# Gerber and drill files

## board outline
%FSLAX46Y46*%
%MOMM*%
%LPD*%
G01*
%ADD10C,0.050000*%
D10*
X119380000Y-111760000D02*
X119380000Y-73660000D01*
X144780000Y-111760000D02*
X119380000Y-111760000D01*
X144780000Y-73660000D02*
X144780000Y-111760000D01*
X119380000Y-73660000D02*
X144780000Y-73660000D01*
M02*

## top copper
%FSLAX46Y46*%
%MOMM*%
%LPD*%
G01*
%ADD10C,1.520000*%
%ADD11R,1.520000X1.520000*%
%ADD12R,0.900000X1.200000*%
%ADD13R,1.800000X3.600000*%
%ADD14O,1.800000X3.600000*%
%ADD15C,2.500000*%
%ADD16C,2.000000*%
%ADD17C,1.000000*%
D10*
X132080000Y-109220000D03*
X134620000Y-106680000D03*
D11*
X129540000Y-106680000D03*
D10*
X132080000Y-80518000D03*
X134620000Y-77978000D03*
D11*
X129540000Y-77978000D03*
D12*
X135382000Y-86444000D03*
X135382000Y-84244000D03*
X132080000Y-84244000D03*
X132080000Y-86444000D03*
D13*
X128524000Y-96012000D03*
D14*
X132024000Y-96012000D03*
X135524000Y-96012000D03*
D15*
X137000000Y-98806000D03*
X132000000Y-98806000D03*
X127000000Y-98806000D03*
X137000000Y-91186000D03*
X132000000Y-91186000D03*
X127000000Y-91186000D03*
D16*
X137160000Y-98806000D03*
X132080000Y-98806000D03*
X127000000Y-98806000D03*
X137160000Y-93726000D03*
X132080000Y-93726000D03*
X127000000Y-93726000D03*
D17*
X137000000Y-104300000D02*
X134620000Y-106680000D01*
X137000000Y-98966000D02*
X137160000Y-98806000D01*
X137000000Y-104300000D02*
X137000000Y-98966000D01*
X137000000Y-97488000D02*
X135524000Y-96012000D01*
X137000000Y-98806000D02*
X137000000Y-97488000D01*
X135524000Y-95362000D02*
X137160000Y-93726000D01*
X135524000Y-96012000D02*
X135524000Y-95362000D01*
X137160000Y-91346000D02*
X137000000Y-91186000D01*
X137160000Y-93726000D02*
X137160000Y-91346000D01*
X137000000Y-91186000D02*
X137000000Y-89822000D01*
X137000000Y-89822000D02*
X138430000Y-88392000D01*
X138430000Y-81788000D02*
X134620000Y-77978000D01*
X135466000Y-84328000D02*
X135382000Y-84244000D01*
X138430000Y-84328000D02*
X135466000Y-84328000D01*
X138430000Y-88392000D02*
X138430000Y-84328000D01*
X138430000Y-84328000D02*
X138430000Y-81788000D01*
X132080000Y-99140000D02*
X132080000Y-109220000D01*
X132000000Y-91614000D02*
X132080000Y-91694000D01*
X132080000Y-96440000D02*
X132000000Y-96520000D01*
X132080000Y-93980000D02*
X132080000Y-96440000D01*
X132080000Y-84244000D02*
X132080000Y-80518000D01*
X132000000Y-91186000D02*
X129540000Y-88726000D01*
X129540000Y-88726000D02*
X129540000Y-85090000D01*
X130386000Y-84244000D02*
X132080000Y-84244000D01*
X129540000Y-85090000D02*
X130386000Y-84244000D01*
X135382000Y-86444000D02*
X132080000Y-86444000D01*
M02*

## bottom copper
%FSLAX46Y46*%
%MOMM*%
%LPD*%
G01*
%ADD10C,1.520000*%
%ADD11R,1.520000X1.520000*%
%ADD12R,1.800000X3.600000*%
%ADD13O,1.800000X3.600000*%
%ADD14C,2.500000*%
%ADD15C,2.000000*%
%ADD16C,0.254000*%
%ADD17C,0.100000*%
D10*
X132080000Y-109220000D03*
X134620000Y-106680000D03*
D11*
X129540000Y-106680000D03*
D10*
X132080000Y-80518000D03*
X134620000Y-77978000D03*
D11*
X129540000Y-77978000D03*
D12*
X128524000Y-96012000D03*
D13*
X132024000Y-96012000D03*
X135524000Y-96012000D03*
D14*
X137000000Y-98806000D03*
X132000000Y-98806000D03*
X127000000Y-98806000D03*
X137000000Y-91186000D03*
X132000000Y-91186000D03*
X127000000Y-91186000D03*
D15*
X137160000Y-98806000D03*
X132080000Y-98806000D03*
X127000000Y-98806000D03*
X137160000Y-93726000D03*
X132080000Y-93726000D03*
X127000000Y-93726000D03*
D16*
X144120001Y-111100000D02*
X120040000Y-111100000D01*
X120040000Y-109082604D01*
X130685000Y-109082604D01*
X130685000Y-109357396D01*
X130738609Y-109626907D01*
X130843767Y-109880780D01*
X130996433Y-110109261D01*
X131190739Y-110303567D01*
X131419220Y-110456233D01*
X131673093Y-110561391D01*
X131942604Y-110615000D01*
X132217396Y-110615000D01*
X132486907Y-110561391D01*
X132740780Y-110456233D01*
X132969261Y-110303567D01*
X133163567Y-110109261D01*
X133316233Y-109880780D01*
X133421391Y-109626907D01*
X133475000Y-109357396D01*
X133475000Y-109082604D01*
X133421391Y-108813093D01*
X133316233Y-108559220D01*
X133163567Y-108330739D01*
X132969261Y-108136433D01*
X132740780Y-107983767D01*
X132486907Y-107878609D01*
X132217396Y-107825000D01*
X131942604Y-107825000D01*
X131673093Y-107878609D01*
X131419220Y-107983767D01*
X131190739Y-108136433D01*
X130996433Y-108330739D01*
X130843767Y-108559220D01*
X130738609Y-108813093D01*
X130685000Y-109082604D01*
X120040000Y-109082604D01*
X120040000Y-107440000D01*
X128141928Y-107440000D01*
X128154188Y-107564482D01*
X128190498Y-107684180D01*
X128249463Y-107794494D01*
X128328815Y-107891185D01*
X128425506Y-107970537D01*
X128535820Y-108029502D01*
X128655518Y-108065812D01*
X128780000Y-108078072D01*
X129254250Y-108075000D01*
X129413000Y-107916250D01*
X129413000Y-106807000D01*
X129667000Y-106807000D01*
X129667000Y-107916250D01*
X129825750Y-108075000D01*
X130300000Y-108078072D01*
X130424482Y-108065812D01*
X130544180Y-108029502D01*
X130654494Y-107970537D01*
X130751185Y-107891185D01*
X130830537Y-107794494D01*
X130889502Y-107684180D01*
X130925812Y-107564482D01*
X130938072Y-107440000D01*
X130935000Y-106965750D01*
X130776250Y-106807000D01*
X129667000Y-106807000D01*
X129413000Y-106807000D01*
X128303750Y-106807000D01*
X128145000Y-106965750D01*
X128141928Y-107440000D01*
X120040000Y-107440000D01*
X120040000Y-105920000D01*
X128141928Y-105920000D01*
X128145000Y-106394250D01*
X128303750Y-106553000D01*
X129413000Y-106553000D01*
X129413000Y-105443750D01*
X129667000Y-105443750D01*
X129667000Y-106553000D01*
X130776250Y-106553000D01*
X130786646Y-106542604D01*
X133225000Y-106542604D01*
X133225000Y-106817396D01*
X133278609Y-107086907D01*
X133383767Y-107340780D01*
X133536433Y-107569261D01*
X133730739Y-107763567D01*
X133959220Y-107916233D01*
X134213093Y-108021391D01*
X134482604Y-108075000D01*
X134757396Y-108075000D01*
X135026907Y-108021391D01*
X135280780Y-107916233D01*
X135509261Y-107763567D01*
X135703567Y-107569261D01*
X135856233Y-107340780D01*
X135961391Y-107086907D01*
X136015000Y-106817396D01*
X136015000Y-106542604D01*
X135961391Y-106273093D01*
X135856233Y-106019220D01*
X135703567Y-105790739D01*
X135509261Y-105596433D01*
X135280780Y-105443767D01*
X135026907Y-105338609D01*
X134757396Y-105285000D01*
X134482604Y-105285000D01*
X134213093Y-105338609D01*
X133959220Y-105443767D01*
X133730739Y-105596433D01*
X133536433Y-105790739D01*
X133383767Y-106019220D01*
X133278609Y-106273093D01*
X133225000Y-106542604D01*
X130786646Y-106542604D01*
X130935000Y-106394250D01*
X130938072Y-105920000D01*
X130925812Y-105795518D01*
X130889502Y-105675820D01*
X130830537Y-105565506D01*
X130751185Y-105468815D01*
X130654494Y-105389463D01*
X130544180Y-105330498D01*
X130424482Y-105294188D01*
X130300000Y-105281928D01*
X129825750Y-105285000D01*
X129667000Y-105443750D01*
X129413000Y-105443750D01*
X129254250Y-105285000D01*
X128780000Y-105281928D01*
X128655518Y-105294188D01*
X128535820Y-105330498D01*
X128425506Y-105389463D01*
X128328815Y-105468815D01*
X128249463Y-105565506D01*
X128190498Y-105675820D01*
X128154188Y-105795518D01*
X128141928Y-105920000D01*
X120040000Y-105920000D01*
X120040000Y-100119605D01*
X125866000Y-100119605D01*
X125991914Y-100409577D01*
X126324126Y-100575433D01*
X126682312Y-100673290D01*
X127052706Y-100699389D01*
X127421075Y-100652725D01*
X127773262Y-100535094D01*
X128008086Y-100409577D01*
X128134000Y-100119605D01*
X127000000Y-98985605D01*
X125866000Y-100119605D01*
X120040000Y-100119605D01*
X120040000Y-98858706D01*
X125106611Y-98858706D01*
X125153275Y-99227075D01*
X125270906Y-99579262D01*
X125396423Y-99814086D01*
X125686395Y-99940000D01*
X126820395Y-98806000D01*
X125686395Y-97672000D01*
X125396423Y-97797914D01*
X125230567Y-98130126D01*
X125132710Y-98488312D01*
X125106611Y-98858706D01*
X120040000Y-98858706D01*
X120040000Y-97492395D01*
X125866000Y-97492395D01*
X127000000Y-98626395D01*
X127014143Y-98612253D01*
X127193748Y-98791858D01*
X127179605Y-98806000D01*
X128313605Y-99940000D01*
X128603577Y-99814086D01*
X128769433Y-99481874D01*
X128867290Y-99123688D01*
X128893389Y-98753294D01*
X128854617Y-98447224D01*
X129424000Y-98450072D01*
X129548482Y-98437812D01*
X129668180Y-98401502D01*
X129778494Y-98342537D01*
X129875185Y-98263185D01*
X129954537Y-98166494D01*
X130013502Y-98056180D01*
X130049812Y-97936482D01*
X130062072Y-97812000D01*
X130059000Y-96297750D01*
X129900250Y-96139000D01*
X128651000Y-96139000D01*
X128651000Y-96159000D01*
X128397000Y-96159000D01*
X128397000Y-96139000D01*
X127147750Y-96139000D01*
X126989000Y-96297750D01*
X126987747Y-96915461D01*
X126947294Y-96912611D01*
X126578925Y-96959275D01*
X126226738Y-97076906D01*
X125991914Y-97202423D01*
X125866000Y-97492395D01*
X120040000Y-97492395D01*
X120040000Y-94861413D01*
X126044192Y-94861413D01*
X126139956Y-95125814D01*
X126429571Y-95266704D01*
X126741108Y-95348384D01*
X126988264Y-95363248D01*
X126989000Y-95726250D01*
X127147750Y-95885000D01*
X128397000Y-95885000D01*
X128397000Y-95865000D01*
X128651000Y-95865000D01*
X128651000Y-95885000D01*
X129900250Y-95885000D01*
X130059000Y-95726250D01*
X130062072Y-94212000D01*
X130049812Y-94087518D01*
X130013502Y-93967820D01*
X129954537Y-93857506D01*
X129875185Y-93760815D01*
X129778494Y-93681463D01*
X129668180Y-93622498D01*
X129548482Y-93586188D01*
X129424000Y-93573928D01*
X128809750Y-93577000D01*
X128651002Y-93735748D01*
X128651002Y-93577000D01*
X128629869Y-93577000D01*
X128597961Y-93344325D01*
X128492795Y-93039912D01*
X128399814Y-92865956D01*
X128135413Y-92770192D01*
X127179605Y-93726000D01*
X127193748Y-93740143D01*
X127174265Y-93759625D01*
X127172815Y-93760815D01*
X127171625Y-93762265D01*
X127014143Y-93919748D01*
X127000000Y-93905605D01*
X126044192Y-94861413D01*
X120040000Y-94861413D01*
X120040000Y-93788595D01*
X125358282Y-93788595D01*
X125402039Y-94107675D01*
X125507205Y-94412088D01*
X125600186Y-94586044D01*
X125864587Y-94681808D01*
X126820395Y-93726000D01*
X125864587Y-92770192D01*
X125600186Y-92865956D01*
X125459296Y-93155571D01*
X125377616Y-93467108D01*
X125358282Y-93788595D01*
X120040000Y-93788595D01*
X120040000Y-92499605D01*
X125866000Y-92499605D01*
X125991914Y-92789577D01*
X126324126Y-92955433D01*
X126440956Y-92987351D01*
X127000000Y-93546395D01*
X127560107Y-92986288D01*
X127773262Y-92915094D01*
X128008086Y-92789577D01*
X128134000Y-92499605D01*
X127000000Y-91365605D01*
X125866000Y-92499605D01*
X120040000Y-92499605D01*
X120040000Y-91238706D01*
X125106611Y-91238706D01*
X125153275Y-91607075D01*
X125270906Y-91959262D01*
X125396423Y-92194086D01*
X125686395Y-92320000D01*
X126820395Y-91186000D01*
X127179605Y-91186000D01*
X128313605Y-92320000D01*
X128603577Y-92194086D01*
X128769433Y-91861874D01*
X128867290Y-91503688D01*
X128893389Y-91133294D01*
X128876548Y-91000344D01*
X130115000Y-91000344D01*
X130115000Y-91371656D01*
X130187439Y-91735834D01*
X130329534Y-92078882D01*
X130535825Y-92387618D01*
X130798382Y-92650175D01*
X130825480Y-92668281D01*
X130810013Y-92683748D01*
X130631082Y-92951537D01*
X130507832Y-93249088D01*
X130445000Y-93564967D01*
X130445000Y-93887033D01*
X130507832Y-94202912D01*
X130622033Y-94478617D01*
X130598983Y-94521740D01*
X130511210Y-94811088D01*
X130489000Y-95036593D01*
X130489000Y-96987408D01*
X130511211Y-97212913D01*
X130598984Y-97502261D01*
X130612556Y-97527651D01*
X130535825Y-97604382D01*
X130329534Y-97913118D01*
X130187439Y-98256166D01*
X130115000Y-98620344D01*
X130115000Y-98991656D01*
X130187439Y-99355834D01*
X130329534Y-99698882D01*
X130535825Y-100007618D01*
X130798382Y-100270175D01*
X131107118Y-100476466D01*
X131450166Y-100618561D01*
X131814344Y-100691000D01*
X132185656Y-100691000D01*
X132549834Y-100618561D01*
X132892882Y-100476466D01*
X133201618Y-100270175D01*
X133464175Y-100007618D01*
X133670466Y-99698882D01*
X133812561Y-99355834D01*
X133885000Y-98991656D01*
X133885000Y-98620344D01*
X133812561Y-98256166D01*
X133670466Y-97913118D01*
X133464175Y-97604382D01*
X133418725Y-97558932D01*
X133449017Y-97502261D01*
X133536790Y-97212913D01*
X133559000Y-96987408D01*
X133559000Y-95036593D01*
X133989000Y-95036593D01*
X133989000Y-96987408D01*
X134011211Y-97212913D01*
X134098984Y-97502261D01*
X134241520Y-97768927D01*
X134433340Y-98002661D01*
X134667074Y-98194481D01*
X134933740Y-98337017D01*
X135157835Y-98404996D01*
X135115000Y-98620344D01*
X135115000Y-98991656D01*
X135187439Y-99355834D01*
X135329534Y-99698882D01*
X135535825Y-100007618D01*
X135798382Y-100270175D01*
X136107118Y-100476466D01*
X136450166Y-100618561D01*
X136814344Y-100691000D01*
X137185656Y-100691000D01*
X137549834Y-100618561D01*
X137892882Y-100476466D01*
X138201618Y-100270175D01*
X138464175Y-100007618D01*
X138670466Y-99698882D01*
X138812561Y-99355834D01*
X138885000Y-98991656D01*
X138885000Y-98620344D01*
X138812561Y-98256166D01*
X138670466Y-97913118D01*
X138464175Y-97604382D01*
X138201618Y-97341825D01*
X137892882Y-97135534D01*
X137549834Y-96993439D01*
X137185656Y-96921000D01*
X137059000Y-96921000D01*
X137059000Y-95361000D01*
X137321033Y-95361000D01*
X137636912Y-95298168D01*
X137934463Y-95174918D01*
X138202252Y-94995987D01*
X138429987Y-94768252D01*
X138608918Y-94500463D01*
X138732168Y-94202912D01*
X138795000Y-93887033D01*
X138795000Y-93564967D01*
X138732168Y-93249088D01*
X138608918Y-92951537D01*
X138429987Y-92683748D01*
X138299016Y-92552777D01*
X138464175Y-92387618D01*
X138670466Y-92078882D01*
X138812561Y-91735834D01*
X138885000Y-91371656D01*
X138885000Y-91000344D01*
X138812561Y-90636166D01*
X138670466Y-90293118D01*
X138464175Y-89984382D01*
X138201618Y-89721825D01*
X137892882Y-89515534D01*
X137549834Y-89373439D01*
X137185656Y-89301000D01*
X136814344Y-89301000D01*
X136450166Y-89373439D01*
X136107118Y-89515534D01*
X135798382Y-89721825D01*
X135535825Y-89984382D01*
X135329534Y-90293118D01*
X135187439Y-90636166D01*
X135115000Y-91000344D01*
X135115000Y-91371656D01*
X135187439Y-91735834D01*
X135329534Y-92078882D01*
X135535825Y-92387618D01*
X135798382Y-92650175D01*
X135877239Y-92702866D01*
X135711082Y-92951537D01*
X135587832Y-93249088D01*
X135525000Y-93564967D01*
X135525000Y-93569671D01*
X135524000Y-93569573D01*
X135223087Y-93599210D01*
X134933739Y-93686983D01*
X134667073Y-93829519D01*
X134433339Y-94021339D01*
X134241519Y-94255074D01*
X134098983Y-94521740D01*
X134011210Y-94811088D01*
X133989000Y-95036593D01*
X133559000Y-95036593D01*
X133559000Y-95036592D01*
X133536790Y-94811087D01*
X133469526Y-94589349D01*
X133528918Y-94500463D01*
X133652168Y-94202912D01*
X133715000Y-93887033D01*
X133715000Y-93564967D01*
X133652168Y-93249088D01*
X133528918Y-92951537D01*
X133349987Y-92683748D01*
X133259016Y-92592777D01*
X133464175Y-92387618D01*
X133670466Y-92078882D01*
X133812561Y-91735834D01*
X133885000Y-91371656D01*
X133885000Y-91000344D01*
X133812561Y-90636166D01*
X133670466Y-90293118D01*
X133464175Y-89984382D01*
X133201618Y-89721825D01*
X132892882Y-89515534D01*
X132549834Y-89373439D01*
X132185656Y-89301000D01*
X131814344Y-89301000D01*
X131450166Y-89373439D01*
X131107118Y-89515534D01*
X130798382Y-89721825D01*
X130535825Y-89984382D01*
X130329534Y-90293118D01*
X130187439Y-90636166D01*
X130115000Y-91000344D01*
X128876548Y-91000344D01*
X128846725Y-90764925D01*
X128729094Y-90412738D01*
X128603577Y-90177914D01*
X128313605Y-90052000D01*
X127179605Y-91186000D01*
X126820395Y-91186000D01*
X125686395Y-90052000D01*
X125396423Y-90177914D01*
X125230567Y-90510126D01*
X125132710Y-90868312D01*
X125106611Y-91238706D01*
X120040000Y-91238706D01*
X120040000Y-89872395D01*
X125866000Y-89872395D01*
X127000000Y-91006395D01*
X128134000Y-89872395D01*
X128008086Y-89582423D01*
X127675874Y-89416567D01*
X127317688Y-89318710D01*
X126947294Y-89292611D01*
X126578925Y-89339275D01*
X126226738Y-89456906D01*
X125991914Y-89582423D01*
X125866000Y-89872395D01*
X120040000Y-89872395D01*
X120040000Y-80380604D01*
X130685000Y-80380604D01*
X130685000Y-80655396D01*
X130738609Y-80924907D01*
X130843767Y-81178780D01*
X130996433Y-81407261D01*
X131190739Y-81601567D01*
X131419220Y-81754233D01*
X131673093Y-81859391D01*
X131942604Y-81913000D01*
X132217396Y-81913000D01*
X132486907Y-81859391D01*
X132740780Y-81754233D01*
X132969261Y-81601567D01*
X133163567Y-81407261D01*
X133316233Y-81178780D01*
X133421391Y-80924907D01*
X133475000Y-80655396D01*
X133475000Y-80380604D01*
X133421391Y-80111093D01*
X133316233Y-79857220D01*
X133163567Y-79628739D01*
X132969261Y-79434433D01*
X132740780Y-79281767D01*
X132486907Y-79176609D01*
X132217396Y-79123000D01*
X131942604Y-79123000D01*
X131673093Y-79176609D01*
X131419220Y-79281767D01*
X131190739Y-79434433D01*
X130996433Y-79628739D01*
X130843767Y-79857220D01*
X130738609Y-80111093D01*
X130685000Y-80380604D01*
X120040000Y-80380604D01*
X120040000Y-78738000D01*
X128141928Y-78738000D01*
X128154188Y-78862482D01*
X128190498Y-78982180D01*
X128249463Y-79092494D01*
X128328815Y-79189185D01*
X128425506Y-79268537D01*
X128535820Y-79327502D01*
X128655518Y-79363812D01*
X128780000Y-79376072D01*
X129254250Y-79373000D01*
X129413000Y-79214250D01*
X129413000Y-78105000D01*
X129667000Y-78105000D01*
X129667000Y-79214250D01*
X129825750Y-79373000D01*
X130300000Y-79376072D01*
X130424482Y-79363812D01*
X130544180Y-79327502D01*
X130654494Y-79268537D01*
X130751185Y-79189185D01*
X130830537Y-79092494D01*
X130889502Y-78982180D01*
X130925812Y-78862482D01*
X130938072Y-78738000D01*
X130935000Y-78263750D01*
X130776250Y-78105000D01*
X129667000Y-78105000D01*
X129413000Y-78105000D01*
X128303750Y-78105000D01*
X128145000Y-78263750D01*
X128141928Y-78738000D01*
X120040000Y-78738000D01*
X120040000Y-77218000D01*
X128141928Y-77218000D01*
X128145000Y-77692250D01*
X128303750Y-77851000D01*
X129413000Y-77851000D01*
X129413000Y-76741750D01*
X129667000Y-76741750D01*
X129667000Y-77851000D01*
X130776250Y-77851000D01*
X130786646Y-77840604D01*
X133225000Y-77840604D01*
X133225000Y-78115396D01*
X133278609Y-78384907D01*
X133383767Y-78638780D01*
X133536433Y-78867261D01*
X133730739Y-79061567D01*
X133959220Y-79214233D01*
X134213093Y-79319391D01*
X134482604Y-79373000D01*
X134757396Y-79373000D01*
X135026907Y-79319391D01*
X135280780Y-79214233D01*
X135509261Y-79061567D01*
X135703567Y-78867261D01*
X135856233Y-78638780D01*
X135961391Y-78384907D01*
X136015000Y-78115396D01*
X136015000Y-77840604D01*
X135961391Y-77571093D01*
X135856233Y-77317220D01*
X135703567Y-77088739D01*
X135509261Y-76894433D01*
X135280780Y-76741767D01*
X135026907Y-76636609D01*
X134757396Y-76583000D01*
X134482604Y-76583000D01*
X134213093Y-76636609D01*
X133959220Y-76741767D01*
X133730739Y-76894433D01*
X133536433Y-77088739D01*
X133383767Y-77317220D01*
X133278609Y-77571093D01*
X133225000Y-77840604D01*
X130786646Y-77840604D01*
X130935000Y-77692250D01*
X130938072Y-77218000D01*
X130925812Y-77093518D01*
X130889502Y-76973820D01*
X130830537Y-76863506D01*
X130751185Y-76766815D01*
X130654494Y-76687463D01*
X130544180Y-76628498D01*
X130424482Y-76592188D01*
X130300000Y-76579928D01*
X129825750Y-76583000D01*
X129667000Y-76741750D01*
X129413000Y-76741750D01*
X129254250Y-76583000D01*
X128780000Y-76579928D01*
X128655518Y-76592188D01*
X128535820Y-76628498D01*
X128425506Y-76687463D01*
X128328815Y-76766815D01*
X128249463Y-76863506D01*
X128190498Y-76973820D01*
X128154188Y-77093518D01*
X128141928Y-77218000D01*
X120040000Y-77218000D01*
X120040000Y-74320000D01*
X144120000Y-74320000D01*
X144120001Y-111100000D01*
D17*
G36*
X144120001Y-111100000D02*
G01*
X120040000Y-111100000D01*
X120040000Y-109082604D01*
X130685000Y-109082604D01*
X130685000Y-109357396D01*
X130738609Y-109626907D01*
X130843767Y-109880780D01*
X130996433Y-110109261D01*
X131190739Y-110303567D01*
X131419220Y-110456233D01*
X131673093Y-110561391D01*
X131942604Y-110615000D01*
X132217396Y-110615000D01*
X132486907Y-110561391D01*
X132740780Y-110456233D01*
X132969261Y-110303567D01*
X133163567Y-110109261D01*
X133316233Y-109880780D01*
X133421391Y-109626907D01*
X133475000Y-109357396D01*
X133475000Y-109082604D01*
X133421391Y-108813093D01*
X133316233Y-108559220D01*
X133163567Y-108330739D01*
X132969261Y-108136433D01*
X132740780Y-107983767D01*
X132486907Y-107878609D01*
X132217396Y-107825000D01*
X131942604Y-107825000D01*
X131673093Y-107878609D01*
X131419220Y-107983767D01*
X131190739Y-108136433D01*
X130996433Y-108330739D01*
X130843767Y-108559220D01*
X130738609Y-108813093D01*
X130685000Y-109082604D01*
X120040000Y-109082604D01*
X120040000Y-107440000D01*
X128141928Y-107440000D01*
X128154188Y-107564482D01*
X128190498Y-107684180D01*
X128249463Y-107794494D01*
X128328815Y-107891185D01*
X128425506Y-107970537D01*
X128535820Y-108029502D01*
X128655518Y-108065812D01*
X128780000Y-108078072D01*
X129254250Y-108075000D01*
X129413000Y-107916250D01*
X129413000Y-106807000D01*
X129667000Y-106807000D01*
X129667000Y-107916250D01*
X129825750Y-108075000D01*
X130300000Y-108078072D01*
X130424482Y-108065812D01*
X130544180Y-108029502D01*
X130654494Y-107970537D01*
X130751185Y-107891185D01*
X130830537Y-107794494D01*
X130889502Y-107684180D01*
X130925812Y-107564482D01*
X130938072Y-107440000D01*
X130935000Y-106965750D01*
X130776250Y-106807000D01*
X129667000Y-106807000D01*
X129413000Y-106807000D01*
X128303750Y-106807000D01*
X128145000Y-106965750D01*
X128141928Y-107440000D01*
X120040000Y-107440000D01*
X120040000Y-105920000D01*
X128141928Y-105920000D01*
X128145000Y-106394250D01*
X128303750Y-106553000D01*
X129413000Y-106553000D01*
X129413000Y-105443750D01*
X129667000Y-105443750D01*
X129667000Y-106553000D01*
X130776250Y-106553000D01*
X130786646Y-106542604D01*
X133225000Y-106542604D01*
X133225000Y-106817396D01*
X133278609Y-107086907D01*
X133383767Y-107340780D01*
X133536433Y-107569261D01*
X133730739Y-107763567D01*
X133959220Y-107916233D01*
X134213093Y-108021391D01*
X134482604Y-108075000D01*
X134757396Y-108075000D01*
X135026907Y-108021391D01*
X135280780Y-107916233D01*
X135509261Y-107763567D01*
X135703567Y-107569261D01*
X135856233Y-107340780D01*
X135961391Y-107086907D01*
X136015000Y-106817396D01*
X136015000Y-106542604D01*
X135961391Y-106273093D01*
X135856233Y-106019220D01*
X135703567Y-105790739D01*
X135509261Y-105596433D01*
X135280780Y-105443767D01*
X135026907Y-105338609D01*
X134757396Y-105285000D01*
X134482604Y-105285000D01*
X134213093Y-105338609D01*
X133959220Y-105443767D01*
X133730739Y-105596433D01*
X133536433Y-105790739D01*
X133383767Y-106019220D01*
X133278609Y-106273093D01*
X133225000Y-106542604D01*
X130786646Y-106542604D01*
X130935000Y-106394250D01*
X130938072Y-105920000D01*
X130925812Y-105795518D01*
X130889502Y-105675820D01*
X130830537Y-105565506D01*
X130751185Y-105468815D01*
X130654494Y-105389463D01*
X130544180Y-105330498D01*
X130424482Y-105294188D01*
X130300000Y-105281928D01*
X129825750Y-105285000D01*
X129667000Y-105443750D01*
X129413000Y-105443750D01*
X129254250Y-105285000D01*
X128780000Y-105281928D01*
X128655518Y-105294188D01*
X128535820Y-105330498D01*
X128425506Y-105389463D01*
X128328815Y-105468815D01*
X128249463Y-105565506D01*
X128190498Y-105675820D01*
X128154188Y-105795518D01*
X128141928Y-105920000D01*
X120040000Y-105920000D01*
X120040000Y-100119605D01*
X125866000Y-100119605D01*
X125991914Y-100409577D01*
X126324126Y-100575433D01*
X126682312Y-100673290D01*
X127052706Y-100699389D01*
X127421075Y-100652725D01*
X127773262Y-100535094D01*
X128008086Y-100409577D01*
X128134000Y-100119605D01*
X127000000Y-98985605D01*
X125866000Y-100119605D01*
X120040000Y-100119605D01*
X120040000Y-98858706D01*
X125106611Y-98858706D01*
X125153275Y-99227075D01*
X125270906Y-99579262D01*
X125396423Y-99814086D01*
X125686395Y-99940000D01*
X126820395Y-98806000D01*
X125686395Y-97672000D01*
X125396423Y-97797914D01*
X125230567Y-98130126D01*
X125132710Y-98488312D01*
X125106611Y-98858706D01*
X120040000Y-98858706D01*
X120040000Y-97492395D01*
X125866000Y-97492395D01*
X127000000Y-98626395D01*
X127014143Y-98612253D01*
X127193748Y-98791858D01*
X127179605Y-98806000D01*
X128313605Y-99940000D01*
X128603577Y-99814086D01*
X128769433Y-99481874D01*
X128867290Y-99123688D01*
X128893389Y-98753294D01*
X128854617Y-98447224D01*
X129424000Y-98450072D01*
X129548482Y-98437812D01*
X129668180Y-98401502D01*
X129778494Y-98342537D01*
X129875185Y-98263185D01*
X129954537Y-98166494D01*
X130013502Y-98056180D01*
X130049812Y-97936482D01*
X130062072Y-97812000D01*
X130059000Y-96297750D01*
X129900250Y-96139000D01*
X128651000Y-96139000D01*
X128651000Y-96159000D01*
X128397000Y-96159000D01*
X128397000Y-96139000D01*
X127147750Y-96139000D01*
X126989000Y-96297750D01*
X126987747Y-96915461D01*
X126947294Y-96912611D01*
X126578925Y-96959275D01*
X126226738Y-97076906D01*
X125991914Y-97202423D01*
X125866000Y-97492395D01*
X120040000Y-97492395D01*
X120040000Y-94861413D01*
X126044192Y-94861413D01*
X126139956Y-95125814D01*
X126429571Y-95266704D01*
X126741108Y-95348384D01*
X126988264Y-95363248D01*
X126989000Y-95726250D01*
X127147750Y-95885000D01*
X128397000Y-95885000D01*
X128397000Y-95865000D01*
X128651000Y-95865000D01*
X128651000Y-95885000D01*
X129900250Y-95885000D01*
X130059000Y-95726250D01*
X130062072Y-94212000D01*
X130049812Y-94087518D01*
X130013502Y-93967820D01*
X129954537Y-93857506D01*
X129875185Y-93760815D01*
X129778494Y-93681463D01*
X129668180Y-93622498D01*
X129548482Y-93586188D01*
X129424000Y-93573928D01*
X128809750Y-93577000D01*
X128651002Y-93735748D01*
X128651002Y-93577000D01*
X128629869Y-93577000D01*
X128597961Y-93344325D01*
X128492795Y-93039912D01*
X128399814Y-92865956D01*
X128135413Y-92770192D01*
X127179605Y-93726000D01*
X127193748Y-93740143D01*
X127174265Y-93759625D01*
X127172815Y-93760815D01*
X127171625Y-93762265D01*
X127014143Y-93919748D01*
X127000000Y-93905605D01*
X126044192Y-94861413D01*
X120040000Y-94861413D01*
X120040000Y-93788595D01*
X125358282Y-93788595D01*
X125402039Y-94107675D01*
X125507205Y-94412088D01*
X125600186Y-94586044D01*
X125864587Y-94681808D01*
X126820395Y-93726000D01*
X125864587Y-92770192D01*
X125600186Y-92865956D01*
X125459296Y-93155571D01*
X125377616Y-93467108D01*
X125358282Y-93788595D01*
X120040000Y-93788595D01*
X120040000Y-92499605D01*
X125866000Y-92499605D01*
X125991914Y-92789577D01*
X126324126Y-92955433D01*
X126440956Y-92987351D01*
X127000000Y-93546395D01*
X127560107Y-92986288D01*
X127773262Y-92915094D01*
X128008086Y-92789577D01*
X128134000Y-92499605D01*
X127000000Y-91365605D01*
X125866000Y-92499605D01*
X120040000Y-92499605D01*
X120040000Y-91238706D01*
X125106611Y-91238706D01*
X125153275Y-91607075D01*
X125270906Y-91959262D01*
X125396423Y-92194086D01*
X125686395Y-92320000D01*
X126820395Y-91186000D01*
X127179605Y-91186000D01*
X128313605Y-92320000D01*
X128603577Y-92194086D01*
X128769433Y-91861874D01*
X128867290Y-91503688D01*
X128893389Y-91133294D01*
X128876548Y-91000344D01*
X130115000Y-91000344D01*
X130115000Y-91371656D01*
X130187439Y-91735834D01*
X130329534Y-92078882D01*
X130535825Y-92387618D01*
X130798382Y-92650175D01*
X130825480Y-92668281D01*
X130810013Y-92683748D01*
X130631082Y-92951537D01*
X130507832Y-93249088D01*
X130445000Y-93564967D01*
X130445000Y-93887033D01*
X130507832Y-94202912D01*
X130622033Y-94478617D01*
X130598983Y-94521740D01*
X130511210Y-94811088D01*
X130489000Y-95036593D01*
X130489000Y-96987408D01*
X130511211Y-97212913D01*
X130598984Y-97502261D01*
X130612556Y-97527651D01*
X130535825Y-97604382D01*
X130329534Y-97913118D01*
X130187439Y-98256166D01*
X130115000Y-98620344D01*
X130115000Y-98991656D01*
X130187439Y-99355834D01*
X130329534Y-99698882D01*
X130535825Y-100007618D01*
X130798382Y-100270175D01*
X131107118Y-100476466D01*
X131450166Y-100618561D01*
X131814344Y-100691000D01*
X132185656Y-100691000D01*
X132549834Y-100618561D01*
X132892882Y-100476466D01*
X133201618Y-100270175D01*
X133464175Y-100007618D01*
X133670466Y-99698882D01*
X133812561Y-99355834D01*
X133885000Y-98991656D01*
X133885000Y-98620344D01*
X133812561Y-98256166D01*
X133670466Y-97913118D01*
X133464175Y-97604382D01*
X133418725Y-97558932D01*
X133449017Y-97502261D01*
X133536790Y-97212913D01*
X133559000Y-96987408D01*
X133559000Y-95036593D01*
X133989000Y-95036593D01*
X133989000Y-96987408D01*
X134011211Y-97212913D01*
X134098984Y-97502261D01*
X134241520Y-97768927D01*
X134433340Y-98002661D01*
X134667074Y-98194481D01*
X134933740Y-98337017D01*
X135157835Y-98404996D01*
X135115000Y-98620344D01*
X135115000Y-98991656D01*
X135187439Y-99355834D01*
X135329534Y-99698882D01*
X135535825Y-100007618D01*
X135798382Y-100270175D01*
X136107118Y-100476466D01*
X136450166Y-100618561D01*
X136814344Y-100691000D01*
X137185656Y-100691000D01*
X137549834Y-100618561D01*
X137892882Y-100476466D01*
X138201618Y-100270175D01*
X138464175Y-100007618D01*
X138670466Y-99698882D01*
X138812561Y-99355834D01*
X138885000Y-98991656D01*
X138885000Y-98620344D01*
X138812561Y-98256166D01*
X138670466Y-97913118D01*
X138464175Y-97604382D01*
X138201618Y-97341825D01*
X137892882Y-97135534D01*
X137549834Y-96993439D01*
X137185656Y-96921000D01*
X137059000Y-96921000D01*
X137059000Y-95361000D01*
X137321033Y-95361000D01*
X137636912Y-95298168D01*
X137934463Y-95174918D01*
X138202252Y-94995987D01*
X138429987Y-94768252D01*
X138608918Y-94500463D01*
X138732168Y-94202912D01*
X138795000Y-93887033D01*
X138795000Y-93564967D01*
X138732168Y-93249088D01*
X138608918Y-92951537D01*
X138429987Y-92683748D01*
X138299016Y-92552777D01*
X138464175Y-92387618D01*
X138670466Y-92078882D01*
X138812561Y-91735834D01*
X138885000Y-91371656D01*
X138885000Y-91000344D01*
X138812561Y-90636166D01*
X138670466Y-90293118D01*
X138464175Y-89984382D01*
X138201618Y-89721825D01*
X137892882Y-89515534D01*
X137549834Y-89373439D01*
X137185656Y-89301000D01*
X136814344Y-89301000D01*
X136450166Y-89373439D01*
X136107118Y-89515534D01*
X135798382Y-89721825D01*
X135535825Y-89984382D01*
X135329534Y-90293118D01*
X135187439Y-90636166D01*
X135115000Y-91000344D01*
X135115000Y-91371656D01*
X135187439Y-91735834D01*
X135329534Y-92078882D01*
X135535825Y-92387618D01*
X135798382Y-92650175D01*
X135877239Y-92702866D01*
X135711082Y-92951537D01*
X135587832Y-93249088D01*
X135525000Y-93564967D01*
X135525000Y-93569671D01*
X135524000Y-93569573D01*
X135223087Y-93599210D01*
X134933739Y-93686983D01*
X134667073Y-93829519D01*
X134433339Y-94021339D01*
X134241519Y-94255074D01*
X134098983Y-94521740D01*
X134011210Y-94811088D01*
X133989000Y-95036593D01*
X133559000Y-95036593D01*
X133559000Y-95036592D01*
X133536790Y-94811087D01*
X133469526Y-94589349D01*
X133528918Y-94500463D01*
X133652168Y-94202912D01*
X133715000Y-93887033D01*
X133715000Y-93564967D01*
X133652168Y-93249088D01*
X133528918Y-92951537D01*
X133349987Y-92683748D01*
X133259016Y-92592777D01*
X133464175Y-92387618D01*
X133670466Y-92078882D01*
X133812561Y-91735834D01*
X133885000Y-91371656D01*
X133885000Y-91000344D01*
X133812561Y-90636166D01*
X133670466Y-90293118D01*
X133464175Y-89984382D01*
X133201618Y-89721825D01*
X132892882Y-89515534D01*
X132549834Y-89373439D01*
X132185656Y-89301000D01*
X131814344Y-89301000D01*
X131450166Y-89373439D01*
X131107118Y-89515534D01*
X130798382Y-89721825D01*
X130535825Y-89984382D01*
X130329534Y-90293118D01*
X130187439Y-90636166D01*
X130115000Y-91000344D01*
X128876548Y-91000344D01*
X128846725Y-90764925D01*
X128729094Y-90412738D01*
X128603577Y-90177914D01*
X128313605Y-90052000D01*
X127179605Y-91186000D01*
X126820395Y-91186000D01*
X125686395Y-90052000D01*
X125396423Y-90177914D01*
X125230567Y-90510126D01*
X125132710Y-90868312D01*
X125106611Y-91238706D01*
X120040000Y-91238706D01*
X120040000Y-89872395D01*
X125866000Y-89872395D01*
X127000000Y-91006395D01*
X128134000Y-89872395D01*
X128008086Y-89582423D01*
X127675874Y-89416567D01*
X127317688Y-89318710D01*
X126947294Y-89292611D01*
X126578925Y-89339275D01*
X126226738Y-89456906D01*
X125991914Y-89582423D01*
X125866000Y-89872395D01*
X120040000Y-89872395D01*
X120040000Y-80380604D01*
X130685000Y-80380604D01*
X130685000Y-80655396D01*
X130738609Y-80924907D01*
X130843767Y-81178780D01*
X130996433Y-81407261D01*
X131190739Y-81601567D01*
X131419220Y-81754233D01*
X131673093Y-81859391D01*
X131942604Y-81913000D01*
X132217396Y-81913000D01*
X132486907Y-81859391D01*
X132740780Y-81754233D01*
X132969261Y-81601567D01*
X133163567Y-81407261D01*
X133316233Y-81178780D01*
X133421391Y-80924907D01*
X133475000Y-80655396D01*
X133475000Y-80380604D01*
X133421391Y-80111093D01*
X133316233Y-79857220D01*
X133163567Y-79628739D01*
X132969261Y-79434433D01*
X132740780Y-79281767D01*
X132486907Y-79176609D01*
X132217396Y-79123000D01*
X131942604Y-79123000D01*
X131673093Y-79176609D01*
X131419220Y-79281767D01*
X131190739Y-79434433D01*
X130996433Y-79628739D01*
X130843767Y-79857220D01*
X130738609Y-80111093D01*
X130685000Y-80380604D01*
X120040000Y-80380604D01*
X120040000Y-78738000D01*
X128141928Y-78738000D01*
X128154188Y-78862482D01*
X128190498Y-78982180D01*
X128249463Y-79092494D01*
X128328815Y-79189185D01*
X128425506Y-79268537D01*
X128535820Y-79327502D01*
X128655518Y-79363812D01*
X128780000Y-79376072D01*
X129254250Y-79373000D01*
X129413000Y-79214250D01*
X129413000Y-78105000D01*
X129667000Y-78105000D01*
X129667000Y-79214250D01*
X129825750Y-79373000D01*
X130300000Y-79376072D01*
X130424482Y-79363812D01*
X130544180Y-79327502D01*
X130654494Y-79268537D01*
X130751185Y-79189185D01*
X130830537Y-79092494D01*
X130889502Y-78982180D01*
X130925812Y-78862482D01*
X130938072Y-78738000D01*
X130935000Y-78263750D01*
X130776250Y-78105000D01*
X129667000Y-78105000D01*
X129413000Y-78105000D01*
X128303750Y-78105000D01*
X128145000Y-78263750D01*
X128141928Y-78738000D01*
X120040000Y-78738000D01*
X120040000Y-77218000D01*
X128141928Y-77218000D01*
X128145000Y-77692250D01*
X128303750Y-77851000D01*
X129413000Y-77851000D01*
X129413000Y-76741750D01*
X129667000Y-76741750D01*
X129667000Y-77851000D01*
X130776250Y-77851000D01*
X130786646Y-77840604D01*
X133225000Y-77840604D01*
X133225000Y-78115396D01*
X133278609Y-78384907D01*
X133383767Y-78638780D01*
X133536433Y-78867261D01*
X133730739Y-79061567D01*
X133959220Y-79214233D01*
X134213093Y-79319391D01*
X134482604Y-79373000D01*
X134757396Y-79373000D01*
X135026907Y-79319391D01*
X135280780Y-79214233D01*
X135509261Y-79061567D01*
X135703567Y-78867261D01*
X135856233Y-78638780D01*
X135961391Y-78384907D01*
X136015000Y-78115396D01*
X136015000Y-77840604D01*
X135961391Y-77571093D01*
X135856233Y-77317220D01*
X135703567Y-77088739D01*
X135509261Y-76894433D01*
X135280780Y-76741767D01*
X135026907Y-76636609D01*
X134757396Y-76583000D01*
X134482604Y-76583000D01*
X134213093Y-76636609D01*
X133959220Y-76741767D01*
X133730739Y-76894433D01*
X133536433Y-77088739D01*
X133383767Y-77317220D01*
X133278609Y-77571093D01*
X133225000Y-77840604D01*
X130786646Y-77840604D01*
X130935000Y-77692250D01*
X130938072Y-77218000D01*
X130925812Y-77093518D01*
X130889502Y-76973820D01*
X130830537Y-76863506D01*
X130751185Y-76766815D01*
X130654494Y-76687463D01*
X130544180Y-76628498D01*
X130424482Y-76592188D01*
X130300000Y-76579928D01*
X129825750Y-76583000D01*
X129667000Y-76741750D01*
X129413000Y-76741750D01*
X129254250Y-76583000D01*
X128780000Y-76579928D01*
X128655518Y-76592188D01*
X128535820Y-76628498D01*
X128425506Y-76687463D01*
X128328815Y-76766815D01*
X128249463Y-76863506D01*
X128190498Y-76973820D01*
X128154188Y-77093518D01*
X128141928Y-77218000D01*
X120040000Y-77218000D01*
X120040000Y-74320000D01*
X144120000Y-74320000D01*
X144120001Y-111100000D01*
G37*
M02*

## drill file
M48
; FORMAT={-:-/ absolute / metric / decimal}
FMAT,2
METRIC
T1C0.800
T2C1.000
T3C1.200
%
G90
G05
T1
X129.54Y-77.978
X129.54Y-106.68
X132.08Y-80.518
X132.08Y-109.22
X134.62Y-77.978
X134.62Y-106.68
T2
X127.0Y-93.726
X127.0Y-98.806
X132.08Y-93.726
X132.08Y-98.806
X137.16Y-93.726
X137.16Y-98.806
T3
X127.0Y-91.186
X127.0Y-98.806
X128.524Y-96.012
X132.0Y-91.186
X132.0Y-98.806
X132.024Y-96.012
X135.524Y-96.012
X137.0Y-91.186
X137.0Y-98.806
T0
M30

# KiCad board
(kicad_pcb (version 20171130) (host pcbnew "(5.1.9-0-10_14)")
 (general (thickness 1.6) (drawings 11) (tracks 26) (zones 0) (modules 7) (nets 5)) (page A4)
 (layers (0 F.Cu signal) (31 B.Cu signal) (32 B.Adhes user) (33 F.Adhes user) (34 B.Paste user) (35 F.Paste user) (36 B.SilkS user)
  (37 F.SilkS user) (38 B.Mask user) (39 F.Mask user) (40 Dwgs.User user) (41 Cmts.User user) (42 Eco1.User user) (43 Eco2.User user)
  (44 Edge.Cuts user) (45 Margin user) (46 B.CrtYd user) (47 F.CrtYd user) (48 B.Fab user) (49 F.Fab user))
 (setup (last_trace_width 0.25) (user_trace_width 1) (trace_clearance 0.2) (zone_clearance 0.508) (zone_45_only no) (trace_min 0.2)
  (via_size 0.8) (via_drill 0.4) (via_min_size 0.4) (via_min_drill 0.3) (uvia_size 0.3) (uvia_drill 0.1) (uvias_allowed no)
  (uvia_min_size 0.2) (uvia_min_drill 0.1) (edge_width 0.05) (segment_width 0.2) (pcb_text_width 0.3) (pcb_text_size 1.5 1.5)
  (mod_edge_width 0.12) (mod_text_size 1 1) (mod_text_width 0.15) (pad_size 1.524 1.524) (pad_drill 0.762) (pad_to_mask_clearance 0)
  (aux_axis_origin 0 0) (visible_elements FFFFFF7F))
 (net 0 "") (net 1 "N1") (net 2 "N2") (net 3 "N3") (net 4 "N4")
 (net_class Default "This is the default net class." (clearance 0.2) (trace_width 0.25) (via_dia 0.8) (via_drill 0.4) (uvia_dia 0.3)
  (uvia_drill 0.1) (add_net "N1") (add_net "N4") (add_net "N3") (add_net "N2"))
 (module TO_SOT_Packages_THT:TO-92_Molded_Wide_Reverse (layer F.Cu) (at 129.54 106.68)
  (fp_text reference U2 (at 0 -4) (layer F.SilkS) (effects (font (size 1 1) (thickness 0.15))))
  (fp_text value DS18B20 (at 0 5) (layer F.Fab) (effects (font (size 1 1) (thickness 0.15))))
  (pad 2 thru_hole circle (at 2.54 2.54 90) (size 1.52 1.52) (drill 0.8) (layers *.Cu *.Mask) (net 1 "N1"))
  (pad 3 thru_hole circle (at 5.08 0 90) (size 1.52 1.52) (drill 0.8) (layers *.Cu *.Mask) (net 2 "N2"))
  (pad 1 thru_hole rect (at 0 0 90) (size 1.52 1.52) (drill 0.8) (layers *.Cu *.Mask) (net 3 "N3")))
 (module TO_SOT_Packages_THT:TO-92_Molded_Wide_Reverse (layer F.Cu) (at 129.54 77.978)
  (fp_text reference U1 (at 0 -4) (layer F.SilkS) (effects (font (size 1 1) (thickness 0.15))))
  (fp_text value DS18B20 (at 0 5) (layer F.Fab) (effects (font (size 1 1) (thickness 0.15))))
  (pad 2 thru_hole circle (at 2.54 2.54 90) (size 1.52 1.52) (drill 0.8) (layers *.Cu *.Mask) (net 1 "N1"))
  (pad 3 thru_hole circle (at 5.08 0 90) (size 1.52 1.52) (drill 0.8) (layers *.Cu *.Mask) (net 2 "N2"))
  (pad 1 thru_hole rect (at 0 0 90) (size 1.52 1.52) (drill 0.8) (layers *.Cu *.Mask) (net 3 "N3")))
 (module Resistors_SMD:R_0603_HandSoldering (layer F.Cu) (at 135.382 85.344 90)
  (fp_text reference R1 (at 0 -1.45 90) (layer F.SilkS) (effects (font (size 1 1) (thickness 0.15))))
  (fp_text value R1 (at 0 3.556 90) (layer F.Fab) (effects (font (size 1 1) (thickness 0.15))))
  (pad 1 smd rect (at -1.1 0 90) (size 1.2 0.9) (layers F.Cu F.Paste F.Mask) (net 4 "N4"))
  (pad 2 smd rect (at 1.1 0 90) (size 1.2 0.9) (layers F.Cu F.Paste F.Mask) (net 2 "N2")))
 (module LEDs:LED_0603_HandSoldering (layer F.Cu) (at 132.08 85.344 270)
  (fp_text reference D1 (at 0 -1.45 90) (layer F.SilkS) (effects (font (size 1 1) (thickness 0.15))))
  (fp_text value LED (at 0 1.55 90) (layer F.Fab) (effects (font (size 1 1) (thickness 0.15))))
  (pad 1 smd rect (at -1.1 0 270) (size 1.2 0.9) (layers F.Cu F.Paste F.Mask) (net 1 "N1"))
  (pad 2 smd rect (at 1.1 0 270) (size 1.2 0.9) (layers F.Cu F.Paste F.Mask) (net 4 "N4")))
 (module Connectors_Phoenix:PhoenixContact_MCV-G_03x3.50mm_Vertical (layer F.Cu) (at 128.524 96.012)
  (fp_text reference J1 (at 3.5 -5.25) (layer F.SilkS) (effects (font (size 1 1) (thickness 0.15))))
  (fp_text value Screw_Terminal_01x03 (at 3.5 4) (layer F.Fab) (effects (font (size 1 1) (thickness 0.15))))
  (pad 1 thru_hole rect (at 0 0) (size 1.8 3.6) (drill 1.2) (layers *.Cu *.Mask) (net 3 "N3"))
  (pad 2 thru_hole oval (at 3.5 0) (size 1.8 3.6) (drill 1.2) (layers *.Cu *.Mask) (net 1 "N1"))
  (pad 3 thru_hole oval (at 7 0) (size 1.8 3.6) (drill 1.2) (layers *.Cu *.Mask) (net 2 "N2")))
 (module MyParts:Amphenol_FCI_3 (layer F.Cu) (at 127 91.186)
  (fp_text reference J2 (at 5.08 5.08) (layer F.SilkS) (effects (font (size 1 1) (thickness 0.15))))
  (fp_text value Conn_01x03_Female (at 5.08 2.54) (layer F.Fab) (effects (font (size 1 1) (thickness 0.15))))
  (pad 3 thru_hole circle (at 10 7.62) (size 2.5 2.5) (drill 1.2) (layers *.Cu *.Mask) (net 2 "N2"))
  (pad 2 thru_hole circle (at 5 7.62) (size 2.5 2.5) (drill 1.2) (layers *.Cu *.Mask) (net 1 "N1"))
  (pad 1 thru_hole circle (at 0 7.62) (size 2.5 2.5) (drill 1.2) (layers *.Cu *.Mask) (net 3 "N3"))
  (pad 3 thru_hole circle (at 10 0) (size 2.5 2.5) (drill 1.2) (layers *.Cu *.Mask) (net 2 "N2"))
  (pad 2 thru_hole circle (at 5 0) (size 2.5 2.5) (drill 1.2) (layers *.Cu *.Mask) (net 1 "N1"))
  (pad 1 thru_hole circle (at 0 0) (size 2.5 2.5) (drill 1.2) (layers *.Cu *.Mask) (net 3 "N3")))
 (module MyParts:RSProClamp (layer F.Cu) (at 127 93.726)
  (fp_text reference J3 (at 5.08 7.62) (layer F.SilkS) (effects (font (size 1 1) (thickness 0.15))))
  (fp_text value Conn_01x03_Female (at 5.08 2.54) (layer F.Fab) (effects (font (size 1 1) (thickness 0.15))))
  (pad 3 thru_hole circle (at 10.16 5.08) (size 2 2) (drill 1) (layers *.Cu *.Mask) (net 2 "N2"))
  (pad 2 thru_hole circle (at 5.08 5.08) (size 2 2) (drill 1) (layers *.Cu *.Mask) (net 1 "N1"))
  (pad 1 thru_hole circle (at 0 5.08) (size 2 2) (drill 1) (layers *.Cu *.Mask) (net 3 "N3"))
  (pad 3 thru_hole circle (at 10.16 0) (size 2 2) (drill 1) (layers *.Cu *.Mask) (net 2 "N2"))
  (pad 2 thru_hole circle (at 5.08 0) (size 2 2) (drill 1) (layers *.Cu *.Mask) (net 1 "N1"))
  (pad 1 thru_hole circle (at 0 0) (size 2 2) (drill 1) (layers *.Cu *.Mask) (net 3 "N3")))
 (gr_line (start 119.38 111.76) (end 119.38 73.66) (layer Edge.Cuts) (width 0.05))
 (gr_line (start 144.78 111.76) (end 119.38 111.76) (layer Edge.Cuts) (width 0.05))
 (gr_line (start 144.78 73.66) (end 144.78 111.76) (layer Edge.Cuts) (width 0.05))
 (gr_line (start 119.38 73.66) (end 144.78 73.66) (layer Edge.Cuts) (width 0.05))
 (segment (start 137 104.3) (end 134.62 106.68) (width 1) (layer F.Cu) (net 2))
 (segment (start 137 98.966) (end 137.16 98.806) (width 1) (layer F.Cu) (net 2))
 (segment (start 137 104.3) (end 137 98.966) (width 1) (layer F.Cu) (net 2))
 (segment (start 137 97.488) (end 135.524 96.012) (width 1) (layer F.Cu) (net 2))
 (segment (start 137 98.806) (end 137 97.488) (width 1) (layer F.Cu) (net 2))
 (segment (start 135.524 95.362) (end 137.16 93.726) (width 1) (layer F.Cu) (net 2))
 (segment (start 135.524 96.012) (end 135.524 95.362) (width 1) (layer F.Cu) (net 2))
 (segment (start 137.16 91.346) (end 137 91.186) (width 1) (layer F.Cu) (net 2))
 (segment (start 137.16 93.726) (end 137.16 91.346) (width 1) (layer F.Cu) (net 2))
 (segment (start 137 91.186) (end 137 89.822) (width 1) (layer F.Cu) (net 2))
 (segment (start 137 89.822) (end 138.43 88.392) (width 1) (layer F.Cu) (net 2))
 (segment (start 138.43 81.788) (end 134.62 77.978) (width 1) (layer F.Cu) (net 2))
 (segment (start 135.466 84.328) (end 135.382 84.244) (width 1) (layer F.Cu) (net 2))
 (segment (start 138.43 84.328) (end 135.466 84.328) (width 1) (layer F.Cu) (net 2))
 (segment (start 138.43 88.392) (end 138.43 84.328) (width 1) (layer F.Cu) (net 2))
 (segment (start 138.43 84.328) (end 138.43 81.788) (width 1) (layer F.Cu) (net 2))
 (segment (start 132.08 99.14) (end 132.08 109.22) (width 1) (layer F.Cu) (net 1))
 (segment (start 132 91.614) (end 132.08 91.694) (width 1) (layer F.Cu) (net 1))
 (segment (start 132.08 96.44) (end 132 96.52) (width 1) (layer F.Cu) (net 1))
 (segment (start 132.08 93.98) (end 132.08 96.44) (width 1) (layer F.Cu) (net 1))
 (segment (start 132.08 84.244) (end 132.08 80.518) (width 1) (layer F.Cu) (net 1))
 (segment (start 132 91.186) (end 129.54 88.726) (width 1) (layer F.Cu) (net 1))
 (segment (start 129.54 88.726) (end 129.54 85.09) (width 1) (layer F.Cu) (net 1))
 (segment (start 130.386 84.244) (end 132.08 84.244) (width 1) (layer F.Cu) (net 1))
 (segment (start 129.54 85.09) (end 130.386 84.244) (width 1) (layer F.Cu) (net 1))
 (segment (start 135.382 86.444) (end 132.08 86.444) (width 1) (layer F.Cu) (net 4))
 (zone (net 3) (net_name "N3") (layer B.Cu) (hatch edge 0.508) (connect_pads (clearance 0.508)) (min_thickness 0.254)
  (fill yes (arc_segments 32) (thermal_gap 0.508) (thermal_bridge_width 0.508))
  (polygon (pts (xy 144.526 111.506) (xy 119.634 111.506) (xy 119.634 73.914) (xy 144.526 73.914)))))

